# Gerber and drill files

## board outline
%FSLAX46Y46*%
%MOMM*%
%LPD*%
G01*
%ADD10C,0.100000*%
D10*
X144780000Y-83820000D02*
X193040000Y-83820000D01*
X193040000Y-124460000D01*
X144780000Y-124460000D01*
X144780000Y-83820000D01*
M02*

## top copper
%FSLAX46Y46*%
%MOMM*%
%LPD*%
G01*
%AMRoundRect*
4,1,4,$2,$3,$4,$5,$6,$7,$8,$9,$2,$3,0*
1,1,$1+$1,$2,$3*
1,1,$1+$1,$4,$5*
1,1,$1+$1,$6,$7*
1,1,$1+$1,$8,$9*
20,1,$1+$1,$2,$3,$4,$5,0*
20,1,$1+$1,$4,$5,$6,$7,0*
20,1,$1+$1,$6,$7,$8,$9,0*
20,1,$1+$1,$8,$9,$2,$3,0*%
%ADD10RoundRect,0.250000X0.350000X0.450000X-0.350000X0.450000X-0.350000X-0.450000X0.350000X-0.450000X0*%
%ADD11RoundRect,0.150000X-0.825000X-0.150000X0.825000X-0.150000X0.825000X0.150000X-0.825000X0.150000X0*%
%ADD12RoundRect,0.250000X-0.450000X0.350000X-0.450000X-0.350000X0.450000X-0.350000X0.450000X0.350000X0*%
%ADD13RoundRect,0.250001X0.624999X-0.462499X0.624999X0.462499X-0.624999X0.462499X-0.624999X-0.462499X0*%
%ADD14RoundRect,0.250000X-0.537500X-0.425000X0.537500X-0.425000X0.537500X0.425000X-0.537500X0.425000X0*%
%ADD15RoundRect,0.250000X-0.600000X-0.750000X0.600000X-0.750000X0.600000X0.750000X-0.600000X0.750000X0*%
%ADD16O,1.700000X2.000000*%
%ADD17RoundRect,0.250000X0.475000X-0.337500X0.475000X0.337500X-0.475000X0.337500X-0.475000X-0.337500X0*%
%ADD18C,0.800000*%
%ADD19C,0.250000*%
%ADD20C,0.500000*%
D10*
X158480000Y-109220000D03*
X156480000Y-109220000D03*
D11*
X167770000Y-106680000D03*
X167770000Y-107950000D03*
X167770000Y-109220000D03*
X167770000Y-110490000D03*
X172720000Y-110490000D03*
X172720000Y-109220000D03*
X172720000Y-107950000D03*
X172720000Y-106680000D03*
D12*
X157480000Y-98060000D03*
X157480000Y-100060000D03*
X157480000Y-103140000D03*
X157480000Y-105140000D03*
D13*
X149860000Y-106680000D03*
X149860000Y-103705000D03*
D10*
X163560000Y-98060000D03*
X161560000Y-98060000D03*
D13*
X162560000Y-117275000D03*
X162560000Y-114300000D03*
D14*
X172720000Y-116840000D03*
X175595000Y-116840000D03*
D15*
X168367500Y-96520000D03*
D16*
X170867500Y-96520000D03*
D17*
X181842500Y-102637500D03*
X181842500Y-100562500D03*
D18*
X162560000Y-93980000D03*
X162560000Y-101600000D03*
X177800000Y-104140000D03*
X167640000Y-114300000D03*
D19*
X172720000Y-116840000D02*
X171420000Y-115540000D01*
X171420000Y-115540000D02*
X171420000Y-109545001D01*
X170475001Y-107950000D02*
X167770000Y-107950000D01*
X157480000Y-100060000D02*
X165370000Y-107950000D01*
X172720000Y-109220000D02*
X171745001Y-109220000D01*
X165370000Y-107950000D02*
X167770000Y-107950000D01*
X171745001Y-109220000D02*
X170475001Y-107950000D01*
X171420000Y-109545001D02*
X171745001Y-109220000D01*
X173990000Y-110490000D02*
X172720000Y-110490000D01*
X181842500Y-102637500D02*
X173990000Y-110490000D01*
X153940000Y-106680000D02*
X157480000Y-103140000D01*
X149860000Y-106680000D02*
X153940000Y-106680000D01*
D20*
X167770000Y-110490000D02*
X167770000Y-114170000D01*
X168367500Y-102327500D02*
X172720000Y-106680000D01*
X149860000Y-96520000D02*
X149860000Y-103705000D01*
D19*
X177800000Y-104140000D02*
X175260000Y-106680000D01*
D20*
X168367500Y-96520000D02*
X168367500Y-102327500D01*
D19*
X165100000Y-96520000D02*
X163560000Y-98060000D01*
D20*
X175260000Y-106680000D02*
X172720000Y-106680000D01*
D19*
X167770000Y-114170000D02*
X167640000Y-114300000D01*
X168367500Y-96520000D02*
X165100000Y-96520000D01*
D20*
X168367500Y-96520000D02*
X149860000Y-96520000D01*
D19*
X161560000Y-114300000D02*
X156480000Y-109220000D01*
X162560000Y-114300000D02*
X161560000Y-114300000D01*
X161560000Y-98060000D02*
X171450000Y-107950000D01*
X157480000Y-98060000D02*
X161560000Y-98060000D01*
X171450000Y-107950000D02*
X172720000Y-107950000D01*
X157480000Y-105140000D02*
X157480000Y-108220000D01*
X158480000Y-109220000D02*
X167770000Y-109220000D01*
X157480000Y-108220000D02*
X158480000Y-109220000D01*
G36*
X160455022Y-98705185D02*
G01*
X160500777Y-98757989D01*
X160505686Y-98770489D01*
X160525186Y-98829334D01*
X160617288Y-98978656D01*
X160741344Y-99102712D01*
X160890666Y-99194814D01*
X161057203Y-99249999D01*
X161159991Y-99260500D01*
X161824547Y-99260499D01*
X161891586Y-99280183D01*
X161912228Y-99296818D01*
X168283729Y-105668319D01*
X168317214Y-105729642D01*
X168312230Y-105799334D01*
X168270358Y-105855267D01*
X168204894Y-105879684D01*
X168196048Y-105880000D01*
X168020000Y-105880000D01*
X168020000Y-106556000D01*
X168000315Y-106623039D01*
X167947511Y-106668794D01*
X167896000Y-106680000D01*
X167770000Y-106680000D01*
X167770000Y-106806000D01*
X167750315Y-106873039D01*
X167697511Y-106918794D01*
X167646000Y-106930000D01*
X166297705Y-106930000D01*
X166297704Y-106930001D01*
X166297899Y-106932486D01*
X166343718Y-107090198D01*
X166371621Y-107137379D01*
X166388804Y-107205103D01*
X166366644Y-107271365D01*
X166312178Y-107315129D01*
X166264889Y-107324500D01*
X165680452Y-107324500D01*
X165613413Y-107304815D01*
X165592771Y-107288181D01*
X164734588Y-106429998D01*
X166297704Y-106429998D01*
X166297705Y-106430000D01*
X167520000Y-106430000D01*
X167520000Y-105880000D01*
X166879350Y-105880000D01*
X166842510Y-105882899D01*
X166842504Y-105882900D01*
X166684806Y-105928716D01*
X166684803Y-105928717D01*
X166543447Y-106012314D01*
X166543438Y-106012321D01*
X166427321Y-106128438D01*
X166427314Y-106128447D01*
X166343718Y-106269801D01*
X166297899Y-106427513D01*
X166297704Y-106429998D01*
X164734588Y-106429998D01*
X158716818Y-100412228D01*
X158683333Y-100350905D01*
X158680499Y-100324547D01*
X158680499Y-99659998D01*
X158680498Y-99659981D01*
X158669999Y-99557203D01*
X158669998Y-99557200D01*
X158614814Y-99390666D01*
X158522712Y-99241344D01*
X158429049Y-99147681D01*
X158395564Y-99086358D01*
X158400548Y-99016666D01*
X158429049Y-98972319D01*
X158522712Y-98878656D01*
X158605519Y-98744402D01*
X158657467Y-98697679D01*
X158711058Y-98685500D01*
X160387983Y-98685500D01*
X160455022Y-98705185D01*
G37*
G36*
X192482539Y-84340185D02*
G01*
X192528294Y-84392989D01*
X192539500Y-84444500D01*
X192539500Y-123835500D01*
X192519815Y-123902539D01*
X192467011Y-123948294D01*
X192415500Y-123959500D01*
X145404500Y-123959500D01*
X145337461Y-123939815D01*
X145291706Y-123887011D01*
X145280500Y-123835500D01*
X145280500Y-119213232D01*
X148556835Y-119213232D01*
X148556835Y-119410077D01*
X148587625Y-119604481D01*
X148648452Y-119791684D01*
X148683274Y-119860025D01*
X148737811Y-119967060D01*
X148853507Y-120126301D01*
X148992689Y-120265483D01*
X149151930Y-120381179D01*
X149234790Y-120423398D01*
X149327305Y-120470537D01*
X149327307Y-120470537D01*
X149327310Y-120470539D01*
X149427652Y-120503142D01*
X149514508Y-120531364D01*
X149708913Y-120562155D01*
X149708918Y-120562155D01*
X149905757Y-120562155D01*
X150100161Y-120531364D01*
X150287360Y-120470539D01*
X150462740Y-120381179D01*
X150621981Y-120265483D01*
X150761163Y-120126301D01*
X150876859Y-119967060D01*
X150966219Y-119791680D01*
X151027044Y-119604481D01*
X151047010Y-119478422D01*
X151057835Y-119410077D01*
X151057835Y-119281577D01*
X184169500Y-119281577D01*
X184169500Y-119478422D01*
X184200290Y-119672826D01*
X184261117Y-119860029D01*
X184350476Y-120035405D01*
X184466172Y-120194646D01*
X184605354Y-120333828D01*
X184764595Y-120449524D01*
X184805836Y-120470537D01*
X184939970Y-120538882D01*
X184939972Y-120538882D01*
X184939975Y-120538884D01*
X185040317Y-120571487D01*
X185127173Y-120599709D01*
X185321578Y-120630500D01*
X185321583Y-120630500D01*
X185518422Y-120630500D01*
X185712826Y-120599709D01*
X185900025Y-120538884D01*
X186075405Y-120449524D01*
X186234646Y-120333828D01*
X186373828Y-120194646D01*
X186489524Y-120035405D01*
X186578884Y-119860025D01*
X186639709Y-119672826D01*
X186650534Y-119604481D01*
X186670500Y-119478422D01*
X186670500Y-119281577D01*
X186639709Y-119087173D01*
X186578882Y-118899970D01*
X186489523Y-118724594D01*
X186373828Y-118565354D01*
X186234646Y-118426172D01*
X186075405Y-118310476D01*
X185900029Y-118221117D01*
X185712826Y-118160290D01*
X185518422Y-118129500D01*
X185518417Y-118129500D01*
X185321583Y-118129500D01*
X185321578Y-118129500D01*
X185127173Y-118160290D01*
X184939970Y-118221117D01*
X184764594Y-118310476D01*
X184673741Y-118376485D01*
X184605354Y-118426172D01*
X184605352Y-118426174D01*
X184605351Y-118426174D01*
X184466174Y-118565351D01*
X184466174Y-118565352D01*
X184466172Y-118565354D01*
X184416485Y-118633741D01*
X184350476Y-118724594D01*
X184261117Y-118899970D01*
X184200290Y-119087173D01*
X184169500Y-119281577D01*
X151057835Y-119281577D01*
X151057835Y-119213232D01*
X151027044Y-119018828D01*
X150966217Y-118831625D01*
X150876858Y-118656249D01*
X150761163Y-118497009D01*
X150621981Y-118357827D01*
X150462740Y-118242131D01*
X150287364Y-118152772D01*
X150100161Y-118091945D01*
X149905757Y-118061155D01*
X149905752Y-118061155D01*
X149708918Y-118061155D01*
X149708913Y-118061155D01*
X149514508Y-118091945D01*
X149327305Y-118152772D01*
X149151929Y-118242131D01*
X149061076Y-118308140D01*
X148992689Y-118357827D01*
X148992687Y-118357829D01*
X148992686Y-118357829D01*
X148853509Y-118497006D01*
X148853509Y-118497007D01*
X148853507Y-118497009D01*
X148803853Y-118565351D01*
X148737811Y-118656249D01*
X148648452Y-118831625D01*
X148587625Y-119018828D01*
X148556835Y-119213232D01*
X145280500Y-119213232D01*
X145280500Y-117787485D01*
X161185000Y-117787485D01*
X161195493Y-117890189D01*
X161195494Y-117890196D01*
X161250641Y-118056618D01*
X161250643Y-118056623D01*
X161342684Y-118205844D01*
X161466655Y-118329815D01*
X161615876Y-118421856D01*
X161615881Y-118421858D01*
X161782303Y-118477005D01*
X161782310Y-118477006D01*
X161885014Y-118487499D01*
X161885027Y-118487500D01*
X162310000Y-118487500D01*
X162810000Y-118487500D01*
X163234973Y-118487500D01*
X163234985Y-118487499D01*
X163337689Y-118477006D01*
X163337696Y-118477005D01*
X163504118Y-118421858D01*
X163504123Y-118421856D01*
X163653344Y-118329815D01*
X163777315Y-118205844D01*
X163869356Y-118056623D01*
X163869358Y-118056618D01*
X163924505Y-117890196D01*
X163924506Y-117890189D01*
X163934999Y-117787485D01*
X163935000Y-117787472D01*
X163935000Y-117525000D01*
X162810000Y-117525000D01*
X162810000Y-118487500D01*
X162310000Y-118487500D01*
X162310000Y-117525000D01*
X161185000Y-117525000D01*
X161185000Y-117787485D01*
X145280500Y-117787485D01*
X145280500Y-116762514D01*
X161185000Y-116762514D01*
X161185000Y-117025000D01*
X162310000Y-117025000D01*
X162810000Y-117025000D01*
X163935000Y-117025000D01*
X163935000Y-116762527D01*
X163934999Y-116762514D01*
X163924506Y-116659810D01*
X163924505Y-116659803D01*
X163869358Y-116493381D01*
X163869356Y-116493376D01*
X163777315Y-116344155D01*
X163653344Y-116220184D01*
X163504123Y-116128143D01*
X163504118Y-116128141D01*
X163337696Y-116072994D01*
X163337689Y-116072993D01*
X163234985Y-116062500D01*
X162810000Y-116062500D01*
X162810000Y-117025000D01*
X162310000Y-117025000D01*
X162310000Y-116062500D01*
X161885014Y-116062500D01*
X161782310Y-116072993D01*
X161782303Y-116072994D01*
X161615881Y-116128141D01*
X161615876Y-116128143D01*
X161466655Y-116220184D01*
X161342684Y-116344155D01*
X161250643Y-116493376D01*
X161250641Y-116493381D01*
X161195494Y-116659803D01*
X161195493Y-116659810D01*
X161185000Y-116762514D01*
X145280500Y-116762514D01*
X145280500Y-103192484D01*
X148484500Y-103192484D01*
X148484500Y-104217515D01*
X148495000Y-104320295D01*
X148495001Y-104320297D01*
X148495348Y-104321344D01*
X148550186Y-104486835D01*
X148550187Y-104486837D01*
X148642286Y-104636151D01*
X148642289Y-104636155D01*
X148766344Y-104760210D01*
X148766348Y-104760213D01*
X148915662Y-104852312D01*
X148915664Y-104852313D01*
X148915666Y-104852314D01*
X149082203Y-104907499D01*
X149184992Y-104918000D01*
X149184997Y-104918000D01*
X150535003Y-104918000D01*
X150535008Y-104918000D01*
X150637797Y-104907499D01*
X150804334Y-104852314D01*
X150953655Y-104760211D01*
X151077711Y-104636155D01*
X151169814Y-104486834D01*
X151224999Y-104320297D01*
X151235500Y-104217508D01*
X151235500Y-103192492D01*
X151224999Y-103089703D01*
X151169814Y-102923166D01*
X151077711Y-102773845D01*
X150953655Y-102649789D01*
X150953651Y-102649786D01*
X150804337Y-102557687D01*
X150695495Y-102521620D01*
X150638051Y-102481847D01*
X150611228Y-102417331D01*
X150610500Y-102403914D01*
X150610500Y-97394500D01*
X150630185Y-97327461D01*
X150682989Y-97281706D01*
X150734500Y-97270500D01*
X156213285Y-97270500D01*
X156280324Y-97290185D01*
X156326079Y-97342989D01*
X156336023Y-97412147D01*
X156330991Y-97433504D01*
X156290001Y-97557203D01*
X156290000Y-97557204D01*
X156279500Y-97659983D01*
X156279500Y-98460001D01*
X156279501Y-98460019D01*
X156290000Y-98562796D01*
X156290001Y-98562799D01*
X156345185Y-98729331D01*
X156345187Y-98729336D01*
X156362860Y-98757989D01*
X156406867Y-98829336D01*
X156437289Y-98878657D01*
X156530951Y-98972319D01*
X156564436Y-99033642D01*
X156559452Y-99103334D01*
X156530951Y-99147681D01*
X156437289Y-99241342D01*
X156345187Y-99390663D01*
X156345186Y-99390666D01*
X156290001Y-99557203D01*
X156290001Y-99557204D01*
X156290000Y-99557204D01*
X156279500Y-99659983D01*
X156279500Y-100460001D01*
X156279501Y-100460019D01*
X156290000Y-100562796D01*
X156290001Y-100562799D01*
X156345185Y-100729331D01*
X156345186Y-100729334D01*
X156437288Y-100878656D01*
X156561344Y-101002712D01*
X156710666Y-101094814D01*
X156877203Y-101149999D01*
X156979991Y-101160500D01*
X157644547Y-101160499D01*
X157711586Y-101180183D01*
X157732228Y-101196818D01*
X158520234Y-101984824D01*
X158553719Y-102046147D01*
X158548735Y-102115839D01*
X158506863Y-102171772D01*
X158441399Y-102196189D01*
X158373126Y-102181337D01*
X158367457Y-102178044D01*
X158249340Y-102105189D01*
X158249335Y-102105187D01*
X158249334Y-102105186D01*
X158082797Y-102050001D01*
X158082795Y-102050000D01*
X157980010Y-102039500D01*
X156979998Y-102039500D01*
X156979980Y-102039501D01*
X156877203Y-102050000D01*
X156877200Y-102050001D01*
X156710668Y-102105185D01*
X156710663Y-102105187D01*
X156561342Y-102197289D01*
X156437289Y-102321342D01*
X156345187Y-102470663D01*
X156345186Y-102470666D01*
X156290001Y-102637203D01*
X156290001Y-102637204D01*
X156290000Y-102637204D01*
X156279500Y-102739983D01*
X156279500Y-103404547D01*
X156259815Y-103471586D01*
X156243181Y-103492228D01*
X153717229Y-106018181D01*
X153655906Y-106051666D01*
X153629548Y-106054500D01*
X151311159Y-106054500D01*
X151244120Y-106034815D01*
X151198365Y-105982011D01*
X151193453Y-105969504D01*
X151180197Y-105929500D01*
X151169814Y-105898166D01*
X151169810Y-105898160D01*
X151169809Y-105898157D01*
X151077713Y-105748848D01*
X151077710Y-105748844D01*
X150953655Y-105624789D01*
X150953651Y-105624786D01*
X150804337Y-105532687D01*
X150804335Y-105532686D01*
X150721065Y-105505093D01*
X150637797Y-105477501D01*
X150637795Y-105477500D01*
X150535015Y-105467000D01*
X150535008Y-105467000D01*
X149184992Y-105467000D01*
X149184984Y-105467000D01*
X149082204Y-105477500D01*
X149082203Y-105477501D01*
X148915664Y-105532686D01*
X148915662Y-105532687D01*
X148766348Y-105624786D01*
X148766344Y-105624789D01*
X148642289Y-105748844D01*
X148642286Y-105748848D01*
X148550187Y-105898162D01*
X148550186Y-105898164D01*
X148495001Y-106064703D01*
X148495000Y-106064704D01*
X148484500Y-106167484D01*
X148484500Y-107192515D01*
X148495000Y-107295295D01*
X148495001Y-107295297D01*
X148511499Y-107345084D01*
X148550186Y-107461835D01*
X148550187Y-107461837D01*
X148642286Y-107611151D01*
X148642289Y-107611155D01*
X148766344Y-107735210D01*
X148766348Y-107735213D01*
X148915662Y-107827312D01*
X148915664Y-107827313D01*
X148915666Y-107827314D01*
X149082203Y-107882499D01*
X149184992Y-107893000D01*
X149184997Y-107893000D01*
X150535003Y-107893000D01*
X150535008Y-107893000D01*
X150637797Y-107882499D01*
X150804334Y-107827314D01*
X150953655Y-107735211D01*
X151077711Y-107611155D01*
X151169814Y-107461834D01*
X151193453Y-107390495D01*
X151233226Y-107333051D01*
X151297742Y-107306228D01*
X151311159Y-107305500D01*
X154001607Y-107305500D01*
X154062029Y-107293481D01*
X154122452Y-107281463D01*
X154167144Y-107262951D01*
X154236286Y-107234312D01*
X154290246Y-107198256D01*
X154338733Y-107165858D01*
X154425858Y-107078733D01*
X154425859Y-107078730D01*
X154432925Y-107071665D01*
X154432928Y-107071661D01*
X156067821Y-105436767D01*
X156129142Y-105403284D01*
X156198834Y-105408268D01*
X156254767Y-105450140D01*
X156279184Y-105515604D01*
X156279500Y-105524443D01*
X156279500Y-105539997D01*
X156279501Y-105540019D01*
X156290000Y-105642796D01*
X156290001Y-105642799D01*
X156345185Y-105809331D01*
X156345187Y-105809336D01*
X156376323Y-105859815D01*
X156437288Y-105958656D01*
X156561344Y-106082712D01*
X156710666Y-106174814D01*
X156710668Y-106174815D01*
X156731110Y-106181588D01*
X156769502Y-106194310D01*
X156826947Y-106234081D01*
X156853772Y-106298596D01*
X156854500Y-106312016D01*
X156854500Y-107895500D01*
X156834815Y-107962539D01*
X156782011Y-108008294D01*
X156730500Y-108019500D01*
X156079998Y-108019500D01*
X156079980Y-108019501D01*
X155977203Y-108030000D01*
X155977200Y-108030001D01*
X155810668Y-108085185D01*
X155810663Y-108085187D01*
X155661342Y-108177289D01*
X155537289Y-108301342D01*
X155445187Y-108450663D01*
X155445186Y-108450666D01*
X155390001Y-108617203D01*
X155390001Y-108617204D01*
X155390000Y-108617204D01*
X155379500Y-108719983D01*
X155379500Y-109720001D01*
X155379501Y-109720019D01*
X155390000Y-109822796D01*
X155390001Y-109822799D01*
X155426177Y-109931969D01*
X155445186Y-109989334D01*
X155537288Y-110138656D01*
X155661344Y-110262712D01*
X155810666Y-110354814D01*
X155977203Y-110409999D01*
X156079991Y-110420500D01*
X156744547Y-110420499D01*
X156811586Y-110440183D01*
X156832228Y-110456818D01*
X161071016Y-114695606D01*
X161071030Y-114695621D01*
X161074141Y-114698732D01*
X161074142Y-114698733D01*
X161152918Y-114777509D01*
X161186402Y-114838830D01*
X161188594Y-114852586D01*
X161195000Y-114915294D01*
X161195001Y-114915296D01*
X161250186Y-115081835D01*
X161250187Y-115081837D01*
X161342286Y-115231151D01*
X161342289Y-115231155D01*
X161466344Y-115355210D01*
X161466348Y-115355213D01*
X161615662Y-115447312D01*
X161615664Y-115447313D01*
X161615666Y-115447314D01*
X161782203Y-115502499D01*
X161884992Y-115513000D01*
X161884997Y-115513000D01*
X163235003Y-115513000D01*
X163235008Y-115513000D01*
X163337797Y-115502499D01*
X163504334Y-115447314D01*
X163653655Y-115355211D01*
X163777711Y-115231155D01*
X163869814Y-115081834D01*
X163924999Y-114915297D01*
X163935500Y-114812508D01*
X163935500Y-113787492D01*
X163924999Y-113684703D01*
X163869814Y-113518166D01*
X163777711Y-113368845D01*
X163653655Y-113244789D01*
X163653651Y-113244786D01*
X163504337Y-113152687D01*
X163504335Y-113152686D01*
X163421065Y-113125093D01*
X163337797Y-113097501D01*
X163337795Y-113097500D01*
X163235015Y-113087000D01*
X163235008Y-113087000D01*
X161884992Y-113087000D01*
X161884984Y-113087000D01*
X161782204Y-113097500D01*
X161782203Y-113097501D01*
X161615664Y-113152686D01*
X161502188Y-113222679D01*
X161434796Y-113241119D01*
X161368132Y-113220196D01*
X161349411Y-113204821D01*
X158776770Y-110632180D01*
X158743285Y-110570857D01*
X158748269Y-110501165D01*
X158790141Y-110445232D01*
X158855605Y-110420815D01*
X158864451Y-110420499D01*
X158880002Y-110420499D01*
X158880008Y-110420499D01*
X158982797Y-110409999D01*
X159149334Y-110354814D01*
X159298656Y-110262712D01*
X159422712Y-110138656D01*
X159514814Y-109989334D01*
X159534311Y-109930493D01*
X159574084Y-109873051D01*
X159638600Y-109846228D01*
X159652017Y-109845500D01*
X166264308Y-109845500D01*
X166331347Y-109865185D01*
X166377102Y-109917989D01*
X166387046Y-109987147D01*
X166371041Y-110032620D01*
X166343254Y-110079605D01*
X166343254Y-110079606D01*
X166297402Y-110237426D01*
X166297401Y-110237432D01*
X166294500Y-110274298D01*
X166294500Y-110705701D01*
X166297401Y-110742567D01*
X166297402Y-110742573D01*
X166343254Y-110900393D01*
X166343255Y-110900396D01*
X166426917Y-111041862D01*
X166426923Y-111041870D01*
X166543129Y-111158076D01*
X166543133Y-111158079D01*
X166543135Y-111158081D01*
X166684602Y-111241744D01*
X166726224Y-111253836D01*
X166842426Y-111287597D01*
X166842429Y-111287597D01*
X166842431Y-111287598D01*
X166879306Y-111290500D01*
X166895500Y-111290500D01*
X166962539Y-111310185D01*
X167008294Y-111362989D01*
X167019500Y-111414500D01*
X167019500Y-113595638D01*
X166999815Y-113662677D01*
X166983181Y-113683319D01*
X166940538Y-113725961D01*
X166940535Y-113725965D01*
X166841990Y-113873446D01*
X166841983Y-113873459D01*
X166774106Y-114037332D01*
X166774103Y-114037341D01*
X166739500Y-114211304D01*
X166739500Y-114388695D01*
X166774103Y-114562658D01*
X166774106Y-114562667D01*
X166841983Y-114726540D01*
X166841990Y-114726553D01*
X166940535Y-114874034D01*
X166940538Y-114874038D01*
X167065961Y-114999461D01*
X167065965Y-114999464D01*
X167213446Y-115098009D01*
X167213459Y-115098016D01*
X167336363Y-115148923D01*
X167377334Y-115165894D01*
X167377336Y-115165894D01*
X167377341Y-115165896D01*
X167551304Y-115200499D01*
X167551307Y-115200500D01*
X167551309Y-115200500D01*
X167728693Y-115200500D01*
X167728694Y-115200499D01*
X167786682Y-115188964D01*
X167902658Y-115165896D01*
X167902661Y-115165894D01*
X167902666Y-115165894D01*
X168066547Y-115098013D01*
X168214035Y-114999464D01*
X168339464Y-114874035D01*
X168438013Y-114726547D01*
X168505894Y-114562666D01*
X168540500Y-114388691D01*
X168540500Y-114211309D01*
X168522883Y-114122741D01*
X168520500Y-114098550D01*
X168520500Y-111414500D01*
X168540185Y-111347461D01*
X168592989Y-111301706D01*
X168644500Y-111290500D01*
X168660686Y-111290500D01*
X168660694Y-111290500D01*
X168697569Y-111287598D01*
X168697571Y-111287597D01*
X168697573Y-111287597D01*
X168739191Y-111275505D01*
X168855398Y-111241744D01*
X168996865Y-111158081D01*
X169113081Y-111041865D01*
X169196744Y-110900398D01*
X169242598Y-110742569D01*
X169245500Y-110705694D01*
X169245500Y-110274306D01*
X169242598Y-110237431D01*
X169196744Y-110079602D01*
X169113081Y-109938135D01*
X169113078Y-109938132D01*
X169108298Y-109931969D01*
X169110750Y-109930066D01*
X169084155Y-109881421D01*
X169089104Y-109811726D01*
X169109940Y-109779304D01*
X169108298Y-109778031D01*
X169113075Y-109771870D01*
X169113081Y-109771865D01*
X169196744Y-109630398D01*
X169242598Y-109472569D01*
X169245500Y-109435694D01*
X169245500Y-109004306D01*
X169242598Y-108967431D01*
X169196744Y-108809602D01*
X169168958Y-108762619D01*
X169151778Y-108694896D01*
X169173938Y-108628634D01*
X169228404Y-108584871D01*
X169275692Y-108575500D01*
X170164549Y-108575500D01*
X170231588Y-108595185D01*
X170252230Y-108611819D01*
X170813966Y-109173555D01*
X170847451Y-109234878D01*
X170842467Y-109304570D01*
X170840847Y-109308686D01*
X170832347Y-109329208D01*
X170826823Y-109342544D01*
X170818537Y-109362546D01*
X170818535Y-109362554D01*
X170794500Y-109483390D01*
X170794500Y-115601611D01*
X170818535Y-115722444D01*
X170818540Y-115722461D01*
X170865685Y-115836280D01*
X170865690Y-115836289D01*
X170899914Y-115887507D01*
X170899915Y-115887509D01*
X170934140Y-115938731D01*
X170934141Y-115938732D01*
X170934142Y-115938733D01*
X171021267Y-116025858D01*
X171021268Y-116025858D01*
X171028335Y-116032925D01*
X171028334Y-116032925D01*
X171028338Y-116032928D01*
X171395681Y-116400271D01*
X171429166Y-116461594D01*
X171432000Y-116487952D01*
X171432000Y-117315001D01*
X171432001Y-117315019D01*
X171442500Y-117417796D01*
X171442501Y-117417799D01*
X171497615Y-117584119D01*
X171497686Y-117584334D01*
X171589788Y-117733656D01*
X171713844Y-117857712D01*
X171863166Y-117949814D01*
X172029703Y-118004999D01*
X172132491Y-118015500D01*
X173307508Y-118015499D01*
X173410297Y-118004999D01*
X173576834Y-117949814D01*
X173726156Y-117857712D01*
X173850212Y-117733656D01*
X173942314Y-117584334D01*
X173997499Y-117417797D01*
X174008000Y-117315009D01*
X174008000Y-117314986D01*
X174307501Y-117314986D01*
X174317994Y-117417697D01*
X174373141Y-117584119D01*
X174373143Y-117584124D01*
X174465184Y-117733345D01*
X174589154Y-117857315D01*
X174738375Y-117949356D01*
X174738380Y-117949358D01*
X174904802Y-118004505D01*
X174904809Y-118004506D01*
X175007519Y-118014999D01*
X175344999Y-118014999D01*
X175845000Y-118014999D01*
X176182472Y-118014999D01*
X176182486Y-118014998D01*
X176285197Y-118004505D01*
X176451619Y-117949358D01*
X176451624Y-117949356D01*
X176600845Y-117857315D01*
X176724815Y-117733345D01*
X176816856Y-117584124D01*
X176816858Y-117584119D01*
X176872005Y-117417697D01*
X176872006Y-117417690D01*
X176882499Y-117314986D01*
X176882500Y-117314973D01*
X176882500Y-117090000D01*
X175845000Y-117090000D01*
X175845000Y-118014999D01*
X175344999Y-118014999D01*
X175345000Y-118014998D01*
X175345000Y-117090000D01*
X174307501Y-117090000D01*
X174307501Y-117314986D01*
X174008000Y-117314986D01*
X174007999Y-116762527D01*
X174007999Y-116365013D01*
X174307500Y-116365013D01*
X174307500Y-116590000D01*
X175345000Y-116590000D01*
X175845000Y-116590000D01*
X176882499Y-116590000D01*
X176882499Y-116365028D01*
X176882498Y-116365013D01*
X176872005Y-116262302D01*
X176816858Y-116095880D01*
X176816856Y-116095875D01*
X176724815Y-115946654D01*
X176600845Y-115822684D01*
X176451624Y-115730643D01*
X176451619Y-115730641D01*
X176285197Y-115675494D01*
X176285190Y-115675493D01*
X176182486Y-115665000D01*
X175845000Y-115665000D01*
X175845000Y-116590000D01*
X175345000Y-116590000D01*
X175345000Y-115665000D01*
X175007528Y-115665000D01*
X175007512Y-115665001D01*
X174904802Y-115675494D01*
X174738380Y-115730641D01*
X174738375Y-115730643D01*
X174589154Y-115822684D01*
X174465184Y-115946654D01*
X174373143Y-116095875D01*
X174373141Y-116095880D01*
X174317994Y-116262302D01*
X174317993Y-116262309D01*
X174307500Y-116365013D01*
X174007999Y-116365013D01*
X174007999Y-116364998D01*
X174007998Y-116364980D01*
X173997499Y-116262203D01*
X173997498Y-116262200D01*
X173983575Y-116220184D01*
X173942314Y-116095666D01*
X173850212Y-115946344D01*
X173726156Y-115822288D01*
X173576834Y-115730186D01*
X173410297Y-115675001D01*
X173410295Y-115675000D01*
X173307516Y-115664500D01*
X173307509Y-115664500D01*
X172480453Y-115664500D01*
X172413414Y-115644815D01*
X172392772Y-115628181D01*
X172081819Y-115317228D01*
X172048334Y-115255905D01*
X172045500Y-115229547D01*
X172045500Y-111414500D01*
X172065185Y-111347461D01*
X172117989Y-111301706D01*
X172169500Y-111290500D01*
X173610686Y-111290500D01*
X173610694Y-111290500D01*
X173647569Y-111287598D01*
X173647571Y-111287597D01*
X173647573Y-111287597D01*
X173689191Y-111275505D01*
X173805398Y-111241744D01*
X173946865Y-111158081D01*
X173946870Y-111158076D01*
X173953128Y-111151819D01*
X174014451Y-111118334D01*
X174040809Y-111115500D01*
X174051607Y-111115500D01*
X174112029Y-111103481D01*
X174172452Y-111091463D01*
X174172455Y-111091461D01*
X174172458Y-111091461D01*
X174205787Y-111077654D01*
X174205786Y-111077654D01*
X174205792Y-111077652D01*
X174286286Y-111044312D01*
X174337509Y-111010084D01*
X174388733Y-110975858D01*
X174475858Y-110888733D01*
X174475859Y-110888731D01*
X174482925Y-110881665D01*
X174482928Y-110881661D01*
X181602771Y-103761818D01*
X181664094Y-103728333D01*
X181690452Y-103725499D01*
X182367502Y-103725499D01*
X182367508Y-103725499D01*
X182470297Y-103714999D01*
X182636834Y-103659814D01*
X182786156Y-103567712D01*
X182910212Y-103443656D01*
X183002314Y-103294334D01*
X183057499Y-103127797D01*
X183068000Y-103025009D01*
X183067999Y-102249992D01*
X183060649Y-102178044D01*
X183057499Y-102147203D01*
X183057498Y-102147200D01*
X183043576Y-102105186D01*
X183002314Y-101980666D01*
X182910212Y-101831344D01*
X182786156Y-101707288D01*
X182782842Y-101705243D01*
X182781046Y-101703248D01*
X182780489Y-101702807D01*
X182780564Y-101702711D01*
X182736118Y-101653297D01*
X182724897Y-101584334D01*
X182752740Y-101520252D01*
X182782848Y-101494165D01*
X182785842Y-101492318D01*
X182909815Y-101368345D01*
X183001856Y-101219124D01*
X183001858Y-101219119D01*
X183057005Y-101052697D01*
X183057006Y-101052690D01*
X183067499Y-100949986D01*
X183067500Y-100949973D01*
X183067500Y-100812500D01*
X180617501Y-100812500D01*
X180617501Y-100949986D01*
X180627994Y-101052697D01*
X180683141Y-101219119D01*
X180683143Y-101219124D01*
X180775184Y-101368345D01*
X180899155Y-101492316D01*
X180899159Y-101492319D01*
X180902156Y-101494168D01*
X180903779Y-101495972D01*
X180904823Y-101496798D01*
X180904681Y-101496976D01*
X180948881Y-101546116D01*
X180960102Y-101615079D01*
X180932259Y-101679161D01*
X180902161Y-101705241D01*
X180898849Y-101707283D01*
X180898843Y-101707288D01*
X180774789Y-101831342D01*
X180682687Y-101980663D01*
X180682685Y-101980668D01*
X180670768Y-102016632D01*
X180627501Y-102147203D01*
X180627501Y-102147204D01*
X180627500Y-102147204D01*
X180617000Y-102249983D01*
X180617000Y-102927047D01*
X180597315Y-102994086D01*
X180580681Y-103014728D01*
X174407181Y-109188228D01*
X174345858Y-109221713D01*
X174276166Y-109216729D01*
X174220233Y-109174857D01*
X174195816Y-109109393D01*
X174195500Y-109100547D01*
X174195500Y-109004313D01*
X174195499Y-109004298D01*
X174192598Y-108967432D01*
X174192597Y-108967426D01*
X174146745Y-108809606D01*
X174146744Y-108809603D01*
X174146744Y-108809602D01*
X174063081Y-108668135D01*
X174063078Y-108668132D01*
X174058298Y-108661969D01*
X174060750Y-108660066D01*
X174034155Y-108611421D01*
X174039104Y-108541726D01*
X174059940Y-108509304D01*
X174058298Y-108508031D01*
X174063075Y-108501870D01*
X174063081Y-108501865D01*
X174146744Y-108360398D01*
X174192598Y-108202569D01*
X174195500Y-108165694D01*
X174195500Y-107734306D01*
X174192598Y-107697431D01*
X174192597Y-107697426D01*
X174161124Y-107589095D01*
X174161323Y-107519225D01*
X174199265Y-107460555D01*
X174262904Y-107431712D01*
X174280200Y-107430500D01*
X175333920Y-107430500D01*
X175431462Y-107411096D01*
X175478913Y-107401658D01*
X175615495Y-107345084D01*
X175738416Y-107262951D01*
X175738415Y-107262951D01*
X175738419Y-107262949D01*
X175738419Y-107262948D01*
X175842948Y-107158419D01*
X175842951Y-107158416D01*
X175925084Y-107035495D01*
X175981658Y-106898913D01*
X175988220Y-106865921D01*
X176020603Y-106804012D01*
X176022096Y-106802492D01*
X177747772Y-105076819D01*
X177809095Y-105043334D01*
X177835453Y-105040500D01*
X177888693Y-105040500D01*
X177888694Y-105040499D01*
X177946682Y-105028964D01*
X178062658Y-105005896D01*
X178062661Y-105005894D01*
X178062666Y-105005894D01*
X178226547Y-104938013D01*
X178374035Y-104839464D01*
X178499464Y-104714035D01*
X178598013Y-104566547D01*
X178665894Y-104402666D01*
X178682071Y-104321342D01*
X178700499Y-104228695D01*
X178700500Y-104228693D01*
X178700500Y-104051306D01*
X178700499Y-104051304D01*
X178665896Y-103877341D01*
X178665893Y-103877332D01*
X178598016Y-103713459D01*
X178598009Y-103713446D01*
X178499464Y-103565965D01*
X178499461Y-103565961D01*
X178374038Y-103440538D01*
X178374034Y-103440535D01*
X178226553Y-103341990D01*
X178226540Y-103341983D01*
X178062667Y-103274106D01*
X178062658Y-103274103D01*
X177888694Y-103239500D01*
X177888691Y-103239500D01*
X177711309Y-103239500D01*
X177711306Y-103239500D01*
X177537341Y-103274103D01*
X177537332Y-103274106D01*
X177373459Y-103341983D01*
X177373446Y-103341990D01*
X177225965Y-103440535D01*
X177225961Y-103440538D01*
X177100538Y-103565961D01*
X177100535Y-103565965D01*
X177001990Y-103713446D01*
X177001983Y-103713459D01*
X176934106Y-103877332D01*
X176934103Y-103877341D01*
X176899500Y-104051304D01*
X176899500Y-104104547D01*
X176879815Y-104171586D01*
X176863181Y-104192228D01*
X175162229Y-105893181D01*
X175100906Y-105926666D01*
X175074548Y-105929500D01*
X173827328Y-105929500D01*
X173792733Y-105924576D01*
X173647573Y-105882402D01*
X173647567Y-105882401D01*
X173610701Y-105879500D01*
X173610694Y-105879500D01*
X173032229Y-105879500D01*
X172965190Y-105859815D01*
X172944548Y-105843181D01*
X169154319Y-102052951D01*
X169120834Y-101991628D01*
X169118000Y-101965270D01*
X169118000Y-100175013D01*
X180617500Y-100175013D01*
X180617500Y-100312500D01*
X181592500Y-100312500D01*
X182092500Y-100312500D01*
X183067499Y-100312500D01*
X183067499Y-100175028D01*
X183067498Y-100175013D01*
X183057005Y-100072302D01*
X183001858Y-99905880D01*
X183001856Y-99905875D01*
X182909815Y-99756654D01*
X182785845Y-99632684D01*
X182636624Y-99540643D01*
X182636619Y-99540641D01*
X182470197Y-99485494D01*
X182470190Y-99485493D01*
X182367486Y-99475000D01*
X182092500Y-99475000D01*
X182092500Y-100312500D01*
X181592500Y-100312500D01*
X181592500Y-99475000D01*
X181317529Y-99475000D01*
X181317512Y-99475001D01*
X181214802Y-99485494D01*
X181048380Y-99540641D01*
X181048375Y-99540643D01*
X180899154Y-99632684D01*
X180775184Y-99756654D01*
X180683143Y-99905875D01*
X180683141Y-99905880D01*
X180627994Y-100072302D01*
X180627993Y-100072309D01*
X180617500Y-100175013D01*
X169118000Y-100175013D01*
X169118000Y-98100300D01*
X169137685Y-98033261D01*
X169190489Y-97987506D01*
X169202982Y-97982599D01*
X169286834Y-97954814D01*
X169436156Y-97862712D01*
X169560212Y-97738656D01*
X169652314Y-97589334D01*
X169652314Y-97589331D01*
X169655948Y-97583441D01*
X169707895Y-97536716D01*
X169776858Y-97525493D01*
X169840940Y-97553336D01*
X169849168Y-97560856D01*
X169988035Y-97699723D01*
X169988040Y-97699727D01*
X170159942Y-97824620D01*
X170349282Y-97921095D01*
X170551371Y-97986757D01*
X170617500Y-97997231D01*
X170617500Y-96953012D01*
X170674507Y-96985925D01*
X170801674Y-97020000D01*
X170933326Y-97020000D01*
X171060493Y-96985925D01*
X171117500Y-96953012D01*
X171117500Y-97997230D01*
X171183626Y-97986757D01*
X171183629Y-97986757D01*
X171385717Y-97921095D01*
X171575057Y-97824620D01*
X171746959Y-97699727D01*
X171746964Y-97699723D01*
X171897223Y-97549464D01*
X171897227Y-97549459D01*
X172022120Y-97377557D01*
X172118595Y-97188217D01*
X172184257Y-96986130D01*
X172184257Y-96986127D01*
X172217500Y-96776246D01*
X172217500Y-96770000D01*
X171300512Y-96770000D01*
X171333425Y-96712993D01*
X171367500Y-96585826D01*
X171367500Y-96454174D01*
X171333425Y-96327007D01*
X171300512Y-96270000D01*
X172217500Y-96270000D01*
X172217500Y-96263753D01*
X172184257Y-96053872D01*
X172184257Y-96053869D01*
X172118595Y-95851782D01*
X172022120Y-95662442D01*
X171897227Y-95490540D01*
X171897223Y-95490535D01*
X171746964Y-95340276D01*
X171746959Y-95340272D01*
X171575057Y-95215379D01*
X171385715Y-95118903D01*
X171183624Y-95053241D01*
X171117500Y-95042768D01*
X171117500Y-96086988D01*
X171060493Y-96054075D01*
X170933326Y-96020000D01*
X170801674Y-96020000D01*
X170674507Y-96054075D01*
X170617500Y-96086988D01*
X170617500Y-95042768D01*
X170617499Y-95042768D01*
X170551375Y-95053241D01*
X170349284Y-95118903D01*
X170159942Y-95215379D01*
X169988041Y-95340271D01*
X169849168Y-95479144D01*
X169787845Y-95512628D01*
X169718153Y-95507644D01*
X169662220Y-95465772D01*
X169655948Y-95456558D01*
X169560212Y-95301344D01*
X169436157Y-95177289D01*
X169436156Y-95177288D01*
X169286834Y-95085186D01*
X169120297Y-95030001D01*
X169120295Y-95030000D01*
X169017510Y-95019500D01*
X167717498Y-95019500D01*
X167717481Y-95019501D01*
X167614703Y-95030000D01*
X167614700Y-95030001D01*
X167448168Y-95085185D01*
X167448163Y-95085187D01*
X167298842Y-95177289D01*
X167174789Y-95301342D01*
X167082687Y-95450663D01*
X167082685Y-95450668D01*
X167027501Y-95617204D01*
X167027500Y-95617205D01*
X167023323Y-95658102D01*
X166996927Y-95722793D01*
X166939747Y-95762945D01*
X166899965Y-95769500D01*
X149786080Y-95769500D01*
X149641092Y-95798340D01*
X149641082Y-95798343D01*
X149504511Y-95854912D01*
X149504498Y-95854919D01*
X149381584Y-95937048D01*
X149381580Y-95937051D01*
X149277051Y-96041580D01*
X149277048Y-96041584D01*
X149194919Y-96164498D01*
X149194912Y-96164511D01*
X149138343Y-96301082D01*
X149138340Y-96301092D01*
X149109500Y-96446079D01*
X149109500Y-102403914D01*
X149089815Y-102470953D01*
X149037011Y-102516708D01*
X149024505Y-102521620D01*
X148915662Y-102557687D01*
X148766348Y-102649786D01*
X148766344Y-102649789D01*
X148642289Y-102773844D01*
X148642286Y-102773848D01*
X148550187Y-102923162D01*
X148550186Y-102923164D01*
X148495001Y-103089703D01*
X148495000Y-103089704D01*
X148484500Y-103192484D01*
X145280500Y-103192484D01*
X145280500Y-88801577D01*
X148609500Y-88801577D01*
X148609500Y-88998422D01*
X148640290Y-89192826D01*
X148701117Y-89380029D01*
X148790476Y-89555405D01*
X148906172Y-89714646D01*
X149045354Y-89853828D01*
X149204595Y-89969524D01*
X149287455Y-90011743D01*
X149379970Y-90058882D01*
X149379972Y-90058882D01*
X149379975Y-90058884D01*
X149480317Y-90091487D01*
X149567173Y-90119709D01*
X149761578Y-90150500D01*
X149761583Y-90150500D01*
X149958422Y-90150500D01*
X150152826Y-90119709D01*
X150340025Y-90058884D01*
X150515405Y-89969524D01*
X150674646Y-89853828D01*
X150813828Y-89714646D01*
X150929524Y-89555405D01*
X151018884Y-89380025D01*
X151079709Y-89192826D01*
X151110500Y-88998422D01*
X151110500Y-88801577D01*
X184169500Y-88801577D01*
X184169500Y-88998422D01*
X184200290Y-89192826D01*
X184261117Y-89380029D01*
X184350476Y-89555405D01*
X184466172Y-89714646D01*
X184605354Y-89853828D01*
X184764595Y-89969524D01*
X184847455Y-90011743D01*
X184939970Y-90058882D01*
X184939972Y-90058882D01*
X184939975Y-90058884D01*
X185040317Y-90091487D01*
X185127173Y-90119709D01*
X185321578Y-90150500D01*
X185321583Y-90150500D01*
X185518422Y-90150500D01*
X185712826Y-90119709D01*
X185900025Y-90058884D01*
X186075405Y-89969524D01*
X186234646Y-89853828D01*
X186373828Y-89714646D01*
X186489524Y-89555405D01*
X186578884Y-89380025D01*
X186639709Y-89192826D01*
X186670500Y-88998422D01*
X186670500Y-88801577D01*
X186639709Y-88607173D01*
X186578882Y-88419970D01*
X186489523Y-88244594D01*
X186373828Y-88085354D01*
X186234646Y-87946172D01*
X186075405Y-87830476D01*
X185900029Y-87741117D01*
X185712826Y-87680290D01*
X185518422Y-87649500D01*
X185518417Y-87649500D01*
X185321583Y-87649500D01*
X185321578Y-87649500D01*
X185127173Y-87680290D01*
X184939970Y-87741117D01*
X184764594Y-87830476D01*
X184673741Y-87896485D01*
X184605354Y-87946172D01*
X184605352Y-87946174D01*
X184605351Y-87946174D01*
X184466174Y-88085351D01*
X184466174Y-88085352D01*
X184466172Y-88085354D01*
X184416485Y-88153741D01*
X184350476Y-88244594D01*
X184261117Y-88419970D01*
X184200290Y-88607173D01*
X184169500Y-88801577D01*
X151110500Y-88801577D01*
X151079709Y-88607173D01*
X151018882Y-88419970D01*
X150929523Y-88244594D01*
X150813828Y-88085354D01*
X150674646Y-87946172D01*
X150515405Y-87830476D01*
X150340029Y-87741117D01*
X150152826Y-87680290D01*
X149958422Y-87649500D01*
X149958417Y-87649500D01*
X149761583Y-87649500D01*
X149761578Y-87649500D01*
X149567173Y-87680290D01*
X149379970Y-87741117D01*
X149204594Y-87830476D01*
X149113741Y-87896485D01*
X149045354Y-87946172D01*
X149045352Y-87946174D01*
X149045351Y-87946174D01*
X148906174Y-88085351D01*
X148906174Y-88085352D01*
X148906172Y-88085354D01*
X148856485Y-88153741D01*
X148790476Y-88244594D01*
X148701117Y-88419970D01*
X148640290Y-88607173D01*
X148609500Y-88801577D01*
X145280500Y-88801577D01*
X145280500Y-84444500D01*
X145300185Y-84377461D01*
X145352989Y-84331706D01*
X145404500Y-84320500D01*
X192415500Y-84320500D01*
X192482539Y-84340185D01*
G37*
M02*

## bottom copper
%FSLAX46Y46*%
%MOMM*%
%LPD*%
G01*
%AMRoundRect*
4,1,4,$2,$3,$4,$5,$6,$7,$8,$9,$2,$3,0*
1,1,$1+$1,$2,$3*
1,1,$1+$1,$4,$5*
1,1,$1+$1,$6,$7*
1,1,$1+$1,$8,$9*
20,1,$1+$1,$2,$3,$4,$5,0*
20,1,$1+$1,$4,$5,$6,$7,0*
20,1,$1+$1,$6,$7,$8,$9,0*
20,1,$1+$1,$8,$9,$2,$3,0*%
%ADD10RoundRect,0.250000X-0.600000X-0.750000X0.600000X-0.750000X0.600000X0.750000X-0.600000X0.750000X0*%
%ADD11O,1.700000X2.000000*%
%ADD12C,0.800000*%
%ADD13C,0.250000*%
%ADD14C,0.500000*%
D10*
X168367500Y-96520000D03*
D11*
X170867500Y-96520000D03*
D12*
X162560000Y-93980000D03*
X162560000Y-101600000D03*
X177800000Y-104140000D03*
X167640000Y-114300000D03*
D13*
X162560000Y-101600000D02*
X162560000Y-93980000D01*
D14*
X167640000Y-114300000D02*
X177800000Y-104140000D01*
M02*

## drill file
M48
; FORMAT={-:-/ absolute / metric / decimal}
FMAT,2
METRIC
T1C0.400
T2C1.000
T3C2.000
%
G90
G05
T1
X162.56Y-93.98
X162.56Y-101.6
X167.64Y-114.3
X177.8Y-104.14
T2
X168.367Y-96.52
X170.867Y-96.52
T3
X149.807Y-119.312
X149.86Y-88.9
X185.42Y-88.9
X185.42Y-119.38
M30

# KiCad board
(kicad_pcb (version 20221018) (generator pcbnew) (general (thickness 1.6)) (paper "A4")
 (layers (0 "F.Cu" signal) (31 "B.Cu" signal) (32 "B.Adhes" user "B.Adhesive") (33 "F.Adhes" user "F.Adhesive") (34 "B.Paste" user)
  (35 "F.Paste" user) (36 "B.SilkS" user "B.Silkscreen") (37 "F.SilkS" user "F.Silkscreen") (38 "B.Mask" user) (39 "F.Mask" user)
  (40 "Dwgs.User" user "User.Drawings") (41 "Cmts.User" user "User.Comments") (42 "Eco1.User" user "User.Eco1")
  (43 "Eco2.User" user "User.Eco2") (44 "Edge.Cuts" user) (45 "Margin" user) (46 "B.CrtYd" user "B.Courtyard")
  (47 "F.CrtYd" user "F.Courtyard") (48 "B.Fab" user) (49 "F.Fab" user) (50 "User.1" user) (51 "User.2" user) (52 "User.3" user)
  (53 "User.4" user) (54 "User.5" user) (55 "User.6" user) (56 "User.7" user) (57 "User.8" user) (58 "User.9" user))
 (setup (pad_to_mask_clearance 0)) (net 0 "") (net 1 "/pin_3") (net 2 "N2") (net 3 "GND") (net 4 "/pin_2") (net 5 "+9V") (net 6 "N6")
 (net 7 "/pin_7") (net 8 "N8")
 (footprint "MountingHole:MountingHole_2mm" (layer "F.Cu") (at 185.42 119.38)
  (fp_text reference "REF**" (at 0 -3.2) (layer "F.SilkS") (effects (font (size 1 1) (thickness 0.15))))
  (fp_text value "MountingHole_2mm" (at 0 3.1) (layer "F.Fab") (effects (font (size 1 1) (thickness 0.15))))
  (pad "" np_thru_hole circle (at 0 0) (size 2 2) (drill 2) (layers "F&B.Cu" "*.Mask")))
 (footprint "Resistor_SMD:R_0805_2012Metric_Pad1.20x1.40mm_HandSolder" (layer "F.Cu") (at 157.48 109.22 180)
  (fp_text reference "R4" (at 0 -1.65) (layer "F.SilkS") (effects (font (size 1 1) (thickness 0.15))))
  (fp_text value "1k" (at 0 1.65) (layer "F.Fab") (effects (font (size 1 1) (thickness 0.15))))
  (pad "1" smd roundrect (at -1 0 180) (size 1.2 1.4) (layers "F.Cu" "F.Paste" "F.Mask") (roundrect_rratio 0.208333) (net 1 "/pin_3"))
  (pad "2" smd roundrect (at 1 0 180) (size 1.2 1.4) (layers "F.Cu" "F.Paste" "F.Mask") (roundrect_rratio 0.208333) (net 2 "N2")))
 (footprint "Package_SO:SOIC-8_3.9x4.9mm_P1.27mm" (layer "F.Cu") (at 170.245 108.585)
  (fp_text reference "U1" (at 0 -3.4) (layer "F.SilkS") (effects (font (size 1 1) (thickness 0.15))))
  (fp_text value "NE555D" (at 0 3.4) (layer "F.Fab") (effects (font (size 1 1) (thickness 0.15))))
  (pad "1" smd roundrect (at -2.475 -1.905) (size 1.95 0.6) (layers "F.Cu" "F.Paste" "F.Mask") (roundrect_rratio 0.25) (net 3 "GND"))
  (pad "2" smd roundrect (at -2.475 -0.635) (size 1.95 0.6) (layers "F.Cu" "F.Paste" "F.Mask") (roundrect_rratio 0.25) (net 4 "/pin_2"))
  (pad "3" smd roundrect (at -2.475 0.635) (size 1.95 0.6) (layers "F.Cu" "F.Paste" "F.Mask") (roundrect_rratio 0.25) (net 1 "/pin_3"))
  (pad "4" smd roundrect (at -2.475 1.905) (size 1.95 0.6) (layers "F.Cu" "F.Paste" "F.Mask") (roundrect_rratio 0.25) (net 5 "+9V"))
  (pad "5" smd roundrect (at 2.475 1.905) (size 1.95 0.6) (layers "F.Cu" "F.Paste" "F.Mask") (roundrect_rratio 0.25) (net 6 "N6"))
  (pad "6" smd roundrect (at 2.475 0.635) (size 1.95 0.6) (layers "F.Cu" "F.Paste" "F.Mask") (roundrect_rratio 0.25) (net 4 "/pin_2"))
  (pad "7" smd roundrect (at 2.475 -0.635) (size 1.95 0.6) (layers "F.Cu" "F.Paste" "F.Mask") (roundrect_rratio 0.25) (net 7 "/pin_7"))
  (pad "8" smd roundrect (at 2.475 -1.905) (size 1.95 0.6) (layers "F.Cu" "F.Paste" "F.Mask") (roundrect_rratio 0.25) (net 5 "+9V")))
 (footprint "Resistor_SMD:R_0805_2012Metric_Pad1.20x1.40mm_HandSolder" (layer "F.Cu") (at 157.48 99.06 -90)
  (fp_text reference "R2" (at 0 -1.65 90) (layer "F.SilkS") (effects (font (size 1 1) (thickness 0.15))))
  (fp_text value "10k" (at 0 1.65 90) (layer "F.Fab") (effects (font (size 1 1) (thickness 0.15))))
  (pad "1" smd roundrect (at -1 0 270) (size 1.2 1.4) (layers "F.Cu" "F.Paste" "F.Mask") (roundrect_rratio 0.208333) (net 7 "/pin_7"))
  (pad "2" smd roundrect (at 1 0 270) (size 1.2 1.4) (layers "F.Cu" "F.Paste" "F.Mask") (roundrect_rratio 0.208333) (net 4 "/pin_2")))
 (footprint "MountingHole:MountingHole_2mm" (layer "F.Cu") (at 149.807335 119.311655)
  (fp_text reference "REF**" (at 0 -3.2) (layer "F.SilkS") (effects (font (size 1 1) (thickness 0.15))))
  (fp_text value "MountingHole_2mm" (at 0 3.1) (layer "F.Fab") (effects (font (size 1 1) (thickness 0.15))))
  (pad "" np_thru_hole circle (at 0 0) (size 2 2) (drill 2) (layers "F&B.Cu" "*.Mask")))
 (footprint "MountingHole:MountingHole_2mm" (layer "F.Cu") (at 149.86 88.9)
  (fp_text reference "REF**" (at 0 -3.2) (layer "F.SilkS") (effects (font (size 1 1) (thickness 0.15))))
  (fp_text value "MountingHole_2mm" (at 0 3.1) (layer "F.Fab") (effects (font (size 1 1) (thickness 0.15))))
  (pad "" np_thru_hole circle (at 0 0) (size 2 2) (drill 2) (layers "F&B.Cu" "*.Mask")))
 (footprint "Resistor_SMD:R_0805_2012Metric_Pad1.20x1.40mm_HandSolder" (layer "F.Cu") (at 157.48 104.14 -90)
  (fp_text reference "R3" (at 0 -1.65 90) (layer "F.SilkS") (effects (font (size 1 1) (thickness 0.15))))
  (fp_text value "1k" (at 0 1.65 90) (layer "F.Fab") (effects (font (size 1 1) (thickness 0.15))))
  (pad "1" smd roundrect (at -1 0 270) (size 1.2 1.4) (layers "F.Cu" "F.Paste" "F.Mask") (roundrect_rratio 0.208333) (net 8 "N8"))
  (pad "2" smd roundrect (at 1 0 270) (size 1.2 1.4) (layers "F.Cu" "F.Paste" "F.Mask") (roundrect_rratio 0.208333) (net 1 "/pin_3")))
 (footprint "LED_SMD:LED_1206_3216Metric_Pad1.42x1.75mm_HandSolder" (layer "F.Cu") (at 149.86 105.1925 90)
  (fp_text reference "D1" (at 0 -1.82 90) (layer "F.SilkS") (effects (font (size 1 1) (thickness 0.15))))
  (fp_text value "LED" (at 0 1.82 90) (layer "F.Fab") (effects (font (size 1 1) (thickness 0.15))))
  (pad "1" smd roundrect (at -1.4875 0 90) (size 1.425 1.75) (layers "F.Cu" "F.Paste" "F.Mask") (roundrect_rratio 0.175439) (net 8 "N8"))
  (pad "2" smd roundrect (at 1.4875 0 90) (size 1.425 1.75) (layers "F.Cu" "F.Paste" "F.Mask") (roundrect_rratio 0.175439) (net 5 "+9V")))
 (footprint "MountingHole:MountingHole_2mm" (layer "F.Cu") (at 185.42 88.9)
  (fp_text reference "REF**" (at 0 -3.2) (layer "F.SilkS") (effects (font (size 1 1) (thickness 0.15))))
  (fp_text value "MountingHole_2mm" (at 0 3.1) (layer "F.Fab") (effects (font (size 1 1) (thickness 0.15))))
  (pad "" np_thru_hole circle (at 0 0) (size 2 2) (drill 2) (layers "*.Cu" "*.Mask")))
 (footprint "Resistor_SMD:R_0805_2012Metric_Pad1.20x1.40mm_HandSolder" (layer "F.Cu") (at 162.56 98.06 180)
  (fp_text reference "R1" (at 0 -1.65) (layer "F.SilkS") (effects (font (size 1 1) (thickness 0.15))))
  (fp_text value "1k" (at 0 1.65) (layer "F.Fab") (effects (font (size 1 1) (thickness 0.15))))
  (pad "1" smd roundrect (at -1 0 180) (size 1.2 1.4) (layers "F.Cu" "F.Paste" "F.Mask") (roundrect_rratio 0.208333) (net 5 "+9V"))
  (pad "2" smd roundrect (at 1 0 180) (size 1.2 1.4) (layers "F.Cu" "F.Paste" "F.Mask") (roundrect_rratio 0.208333) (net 7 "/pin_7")))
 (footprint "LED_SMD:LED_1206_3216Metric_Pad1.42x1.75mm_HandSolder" (layer "F.Cu") (at 162.56 115.7875 90)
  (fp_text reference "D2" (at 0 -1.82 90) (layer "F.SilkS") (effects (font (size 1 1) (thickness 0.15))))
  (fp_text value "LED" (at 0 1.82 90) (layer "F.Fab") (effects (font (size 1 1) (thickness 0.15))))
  (pad "1" smd roundrect (at -1.4875 0 90) (size 1.425 1.75) (layers "F.Cu" "F.Paste" "F.Mask") (roundrect_rratio 0.175439) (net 3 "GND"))
  (pad "2" smd roundrect (at 1.4875 0 90) (size 1.425 1.75) (layers "F.Cu" "F.Paste" "F.Mask") (roundrect_rratio 0.175439) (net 2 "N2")))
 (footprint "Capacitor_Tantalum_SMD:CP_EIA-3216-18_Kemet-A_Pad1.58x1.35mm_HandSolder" (layer "F.Cu") (at 174.1575 116.84)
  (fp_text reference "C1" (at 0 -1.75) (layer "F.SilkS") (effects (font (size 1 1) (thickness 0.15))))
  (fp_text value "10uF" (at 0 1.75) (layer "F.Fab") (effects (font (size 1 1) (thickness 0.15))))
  (pad "1" smd roundrect (at -1.4375 0) (size 1.575 1.35) (layers "F.Cu" "F.Paste" "F.Mask") (roundrect_rratio 0.185185) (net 4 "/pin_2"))
  (pad "2" smd roundrect (at 1.4375 0) (size 1.575 1.35) (layers "F.Cu" "F.Paste" "F.Mask") (roundrect_rratio 0.185185) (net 3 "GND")))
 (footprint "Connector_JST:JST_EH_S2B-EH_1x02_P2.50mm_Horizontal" (layer "F.Cu") (at 168.3675 96.52)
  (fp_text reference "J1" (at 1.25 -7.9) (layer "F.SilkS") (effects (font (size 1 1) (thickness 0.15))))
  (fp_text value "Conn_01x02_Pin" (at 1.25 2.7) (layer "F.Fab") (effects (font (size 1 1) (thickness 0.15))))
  (pad "1" thru_hole roundrect (at 0 0) (size 1.7 2) (drill 1) (layers "*.Cu" "*.Mask") (roundrect_rratio 0.147059) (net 5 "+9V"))
  (pad "2" thru_hole oval (at 2.5 0) (size 1.7 2) (drill 1) (layers "*.Cu" "*.Mask") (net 3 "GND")))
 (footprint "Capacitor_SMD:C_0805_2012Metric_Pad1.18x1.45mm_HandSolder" (layer "F.Cu") (at 181.8425 101.6 90)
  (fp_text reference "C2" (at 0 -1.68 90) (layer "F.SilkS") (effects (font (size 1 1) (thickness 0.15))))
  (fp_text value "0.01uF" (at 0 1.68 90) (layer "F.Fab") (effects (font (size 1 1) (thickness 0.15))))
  (pad "1" smd roundrect (at -1.0375 0 90) (size 1.175 1.45) (layers "F.Cu" "F.Paste" "F.Mask") (roundrect_rratio 0.212766) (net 6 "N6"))
  (pad "2" smd roundrect (at 1.0375 0 90) (size 1.175 1.45) (layers "F.Cu" "F.Paste" "F.Mask") (roundrect_rratio 0.212766) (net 3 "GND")))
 (gr_rect (start 144.78 83.82) (end 193.04 124.46) (stroke (width 0.1) (type default)) (fill none) (layer "Edge.Cuts"))
 (segment (start 172.72 116.84) (end 171.42 115.54) (width 0.25) (layer "F.Cu") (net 4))
 (segment (start 171.42 115.54) (end 171.42 109.545001) (width 0.25) (layer "F.Cu") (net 4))
 (segment (start 170.475001 107.95) (end 167.77 107.95) (width 0.25) (layer "F.Cu") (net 4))
 (segment (start 157.48 100.06) (end 165.37 107.95) (width 0.25) (layer "F.Cu") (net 4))
 (segment (start 172.72 109.22) (end 171.745001 109.22) (width 0.25) (layer "F.Cu") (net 4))
 (segment (start 165.37 107.95) (end 167.77 107.95) (width 0.25) (layer "F.Cu") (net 4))
 (segment (start 171.745001 109.22) (end 170.475001 107.95) (width 0.25) (layer "F.Cu") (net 4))
 (segment (start 171.42 109.545001) (end 171.745001 109.22) (width 0.25) (layer "F.Cu") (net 4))
 (via (at 162.56 93.98) (size 0.8) (drill 0.4) (layers "F.Cu" "B.Cu") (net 3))
 (via (at 162.56 101.6) (size 0.8) (drill 0.4) (layers "F.Cu" "B.Cu") (free) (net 3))
 (segment (start 162.56 101.6) (end 162.56 93.98) (width 0.25) (layer "B.Cu") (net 3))
 (segment (start 173.99 110.49) (end 172.72 110.49) (width 0.25) (layer "F.Cu") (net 6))
 (segment (start 181.8425 102.6375) (end 173.99 110.49) (width 0.25) (layer "F.Cu") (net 6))
 (segment (start 153.94 106.68) (end 157.48 103.14) (width 0.25) (layer "F.Cu") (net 8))
 (segment (start 149.86 106.68) (end 153.94 106.68) (width 0.25) (layer "F.Cu") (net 8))
 (segment (start 167.77 110.49) (end 167.77 114.17) (width 0.5) (layer "F.Cu") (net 5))
 (segment (start 168.3675 102.3275) (end 172.72 106.68) (width 0.5) (layer "F.Cu") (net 5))
 (segment (start 149.86 96.52) (end 149.86 103.705) (width 0.5) (layer "F.Cu") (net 5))
 (segment (start 177.8 104.14) (end 175.26 106.68) (width 0.25) (layer "F.Cu") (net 5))
 (segment (start 168.3675 96.52) (end 168.3675 102.3275) (width 0.5) (layer "F.Cu") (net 5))
 (segment (start 165.1 96.52) (end 163.56 98.06) (width 0.25) (layer "F.Cu") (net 5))
 (segment (start 175.26 106.68) (end 172.72 106.68) (width 0.5) (layer "F.Cu") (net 5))
 (segment (start 167.77 114.17) (end 167.64 114.3) (width 0.25) (layer "F.Cu") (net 5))
 (segment (start 168.3675 96.52) (end 165.1 96.52) (width 0.25) (layer "F.Cu") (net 5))
 (segment (start 168.3675 96.52) (end 149.86 96.52) (width 0.5) (layer "F.Cu") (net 5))
 (via (at 177.8 104.14) (size 0.8) (drill 0.4) (layers "F.Cu" "B.Cu") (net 5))
 (via (at 167.64 114.3) (size 0.8) (drill 0.4) (layers "F.Cu" "B.Cu") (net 5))
 (segment (start 167.64 114.3) (end 177.8 104.14) (width 0.5) (layer "B.Cu") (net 5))
 (segment (start 161.56 114.3) (end 156.48 109.22) (width 0.25) (layer "F.Cu") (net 2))
 (segment (start 162.56 114.3) (end 161.56 114.3) (width 0.25) (layer "F.Cu") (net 2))
 (segment (start 161.56 98.06) (end 171.45 107.95) (width 0.25) (layer "F.Cu") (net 7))
 (segment (start 157.48 98.06) (end 161.56 98.06) (width 0.25) (layer "F.Cu") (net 7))
 (segment (start 171.45 107.95) (end 172.72 107.95) (width 0.25) (layer "F.Cu") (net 7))
 (segment (start 157.48 105.14) (end 157.48 108.22) (width 0.25) (layer "F.Cu") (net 1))
 (segment (start 158.48 109.22) (end 167.77 109.22) (width 0.25) (layer "F.Cu") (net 1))
 (segment (start 157.48 108.22) (end 158.48 109.22) (width 0.25) (layer "F.Cu") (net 1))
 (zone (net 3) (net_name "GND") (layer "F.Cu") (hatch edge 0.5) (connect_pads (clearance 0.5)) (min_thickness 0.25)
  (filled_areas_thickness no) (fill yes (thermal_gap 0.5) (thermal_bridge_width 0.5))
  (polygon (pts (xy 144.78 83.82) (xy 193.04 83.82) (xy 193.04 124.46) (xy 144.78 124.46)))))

